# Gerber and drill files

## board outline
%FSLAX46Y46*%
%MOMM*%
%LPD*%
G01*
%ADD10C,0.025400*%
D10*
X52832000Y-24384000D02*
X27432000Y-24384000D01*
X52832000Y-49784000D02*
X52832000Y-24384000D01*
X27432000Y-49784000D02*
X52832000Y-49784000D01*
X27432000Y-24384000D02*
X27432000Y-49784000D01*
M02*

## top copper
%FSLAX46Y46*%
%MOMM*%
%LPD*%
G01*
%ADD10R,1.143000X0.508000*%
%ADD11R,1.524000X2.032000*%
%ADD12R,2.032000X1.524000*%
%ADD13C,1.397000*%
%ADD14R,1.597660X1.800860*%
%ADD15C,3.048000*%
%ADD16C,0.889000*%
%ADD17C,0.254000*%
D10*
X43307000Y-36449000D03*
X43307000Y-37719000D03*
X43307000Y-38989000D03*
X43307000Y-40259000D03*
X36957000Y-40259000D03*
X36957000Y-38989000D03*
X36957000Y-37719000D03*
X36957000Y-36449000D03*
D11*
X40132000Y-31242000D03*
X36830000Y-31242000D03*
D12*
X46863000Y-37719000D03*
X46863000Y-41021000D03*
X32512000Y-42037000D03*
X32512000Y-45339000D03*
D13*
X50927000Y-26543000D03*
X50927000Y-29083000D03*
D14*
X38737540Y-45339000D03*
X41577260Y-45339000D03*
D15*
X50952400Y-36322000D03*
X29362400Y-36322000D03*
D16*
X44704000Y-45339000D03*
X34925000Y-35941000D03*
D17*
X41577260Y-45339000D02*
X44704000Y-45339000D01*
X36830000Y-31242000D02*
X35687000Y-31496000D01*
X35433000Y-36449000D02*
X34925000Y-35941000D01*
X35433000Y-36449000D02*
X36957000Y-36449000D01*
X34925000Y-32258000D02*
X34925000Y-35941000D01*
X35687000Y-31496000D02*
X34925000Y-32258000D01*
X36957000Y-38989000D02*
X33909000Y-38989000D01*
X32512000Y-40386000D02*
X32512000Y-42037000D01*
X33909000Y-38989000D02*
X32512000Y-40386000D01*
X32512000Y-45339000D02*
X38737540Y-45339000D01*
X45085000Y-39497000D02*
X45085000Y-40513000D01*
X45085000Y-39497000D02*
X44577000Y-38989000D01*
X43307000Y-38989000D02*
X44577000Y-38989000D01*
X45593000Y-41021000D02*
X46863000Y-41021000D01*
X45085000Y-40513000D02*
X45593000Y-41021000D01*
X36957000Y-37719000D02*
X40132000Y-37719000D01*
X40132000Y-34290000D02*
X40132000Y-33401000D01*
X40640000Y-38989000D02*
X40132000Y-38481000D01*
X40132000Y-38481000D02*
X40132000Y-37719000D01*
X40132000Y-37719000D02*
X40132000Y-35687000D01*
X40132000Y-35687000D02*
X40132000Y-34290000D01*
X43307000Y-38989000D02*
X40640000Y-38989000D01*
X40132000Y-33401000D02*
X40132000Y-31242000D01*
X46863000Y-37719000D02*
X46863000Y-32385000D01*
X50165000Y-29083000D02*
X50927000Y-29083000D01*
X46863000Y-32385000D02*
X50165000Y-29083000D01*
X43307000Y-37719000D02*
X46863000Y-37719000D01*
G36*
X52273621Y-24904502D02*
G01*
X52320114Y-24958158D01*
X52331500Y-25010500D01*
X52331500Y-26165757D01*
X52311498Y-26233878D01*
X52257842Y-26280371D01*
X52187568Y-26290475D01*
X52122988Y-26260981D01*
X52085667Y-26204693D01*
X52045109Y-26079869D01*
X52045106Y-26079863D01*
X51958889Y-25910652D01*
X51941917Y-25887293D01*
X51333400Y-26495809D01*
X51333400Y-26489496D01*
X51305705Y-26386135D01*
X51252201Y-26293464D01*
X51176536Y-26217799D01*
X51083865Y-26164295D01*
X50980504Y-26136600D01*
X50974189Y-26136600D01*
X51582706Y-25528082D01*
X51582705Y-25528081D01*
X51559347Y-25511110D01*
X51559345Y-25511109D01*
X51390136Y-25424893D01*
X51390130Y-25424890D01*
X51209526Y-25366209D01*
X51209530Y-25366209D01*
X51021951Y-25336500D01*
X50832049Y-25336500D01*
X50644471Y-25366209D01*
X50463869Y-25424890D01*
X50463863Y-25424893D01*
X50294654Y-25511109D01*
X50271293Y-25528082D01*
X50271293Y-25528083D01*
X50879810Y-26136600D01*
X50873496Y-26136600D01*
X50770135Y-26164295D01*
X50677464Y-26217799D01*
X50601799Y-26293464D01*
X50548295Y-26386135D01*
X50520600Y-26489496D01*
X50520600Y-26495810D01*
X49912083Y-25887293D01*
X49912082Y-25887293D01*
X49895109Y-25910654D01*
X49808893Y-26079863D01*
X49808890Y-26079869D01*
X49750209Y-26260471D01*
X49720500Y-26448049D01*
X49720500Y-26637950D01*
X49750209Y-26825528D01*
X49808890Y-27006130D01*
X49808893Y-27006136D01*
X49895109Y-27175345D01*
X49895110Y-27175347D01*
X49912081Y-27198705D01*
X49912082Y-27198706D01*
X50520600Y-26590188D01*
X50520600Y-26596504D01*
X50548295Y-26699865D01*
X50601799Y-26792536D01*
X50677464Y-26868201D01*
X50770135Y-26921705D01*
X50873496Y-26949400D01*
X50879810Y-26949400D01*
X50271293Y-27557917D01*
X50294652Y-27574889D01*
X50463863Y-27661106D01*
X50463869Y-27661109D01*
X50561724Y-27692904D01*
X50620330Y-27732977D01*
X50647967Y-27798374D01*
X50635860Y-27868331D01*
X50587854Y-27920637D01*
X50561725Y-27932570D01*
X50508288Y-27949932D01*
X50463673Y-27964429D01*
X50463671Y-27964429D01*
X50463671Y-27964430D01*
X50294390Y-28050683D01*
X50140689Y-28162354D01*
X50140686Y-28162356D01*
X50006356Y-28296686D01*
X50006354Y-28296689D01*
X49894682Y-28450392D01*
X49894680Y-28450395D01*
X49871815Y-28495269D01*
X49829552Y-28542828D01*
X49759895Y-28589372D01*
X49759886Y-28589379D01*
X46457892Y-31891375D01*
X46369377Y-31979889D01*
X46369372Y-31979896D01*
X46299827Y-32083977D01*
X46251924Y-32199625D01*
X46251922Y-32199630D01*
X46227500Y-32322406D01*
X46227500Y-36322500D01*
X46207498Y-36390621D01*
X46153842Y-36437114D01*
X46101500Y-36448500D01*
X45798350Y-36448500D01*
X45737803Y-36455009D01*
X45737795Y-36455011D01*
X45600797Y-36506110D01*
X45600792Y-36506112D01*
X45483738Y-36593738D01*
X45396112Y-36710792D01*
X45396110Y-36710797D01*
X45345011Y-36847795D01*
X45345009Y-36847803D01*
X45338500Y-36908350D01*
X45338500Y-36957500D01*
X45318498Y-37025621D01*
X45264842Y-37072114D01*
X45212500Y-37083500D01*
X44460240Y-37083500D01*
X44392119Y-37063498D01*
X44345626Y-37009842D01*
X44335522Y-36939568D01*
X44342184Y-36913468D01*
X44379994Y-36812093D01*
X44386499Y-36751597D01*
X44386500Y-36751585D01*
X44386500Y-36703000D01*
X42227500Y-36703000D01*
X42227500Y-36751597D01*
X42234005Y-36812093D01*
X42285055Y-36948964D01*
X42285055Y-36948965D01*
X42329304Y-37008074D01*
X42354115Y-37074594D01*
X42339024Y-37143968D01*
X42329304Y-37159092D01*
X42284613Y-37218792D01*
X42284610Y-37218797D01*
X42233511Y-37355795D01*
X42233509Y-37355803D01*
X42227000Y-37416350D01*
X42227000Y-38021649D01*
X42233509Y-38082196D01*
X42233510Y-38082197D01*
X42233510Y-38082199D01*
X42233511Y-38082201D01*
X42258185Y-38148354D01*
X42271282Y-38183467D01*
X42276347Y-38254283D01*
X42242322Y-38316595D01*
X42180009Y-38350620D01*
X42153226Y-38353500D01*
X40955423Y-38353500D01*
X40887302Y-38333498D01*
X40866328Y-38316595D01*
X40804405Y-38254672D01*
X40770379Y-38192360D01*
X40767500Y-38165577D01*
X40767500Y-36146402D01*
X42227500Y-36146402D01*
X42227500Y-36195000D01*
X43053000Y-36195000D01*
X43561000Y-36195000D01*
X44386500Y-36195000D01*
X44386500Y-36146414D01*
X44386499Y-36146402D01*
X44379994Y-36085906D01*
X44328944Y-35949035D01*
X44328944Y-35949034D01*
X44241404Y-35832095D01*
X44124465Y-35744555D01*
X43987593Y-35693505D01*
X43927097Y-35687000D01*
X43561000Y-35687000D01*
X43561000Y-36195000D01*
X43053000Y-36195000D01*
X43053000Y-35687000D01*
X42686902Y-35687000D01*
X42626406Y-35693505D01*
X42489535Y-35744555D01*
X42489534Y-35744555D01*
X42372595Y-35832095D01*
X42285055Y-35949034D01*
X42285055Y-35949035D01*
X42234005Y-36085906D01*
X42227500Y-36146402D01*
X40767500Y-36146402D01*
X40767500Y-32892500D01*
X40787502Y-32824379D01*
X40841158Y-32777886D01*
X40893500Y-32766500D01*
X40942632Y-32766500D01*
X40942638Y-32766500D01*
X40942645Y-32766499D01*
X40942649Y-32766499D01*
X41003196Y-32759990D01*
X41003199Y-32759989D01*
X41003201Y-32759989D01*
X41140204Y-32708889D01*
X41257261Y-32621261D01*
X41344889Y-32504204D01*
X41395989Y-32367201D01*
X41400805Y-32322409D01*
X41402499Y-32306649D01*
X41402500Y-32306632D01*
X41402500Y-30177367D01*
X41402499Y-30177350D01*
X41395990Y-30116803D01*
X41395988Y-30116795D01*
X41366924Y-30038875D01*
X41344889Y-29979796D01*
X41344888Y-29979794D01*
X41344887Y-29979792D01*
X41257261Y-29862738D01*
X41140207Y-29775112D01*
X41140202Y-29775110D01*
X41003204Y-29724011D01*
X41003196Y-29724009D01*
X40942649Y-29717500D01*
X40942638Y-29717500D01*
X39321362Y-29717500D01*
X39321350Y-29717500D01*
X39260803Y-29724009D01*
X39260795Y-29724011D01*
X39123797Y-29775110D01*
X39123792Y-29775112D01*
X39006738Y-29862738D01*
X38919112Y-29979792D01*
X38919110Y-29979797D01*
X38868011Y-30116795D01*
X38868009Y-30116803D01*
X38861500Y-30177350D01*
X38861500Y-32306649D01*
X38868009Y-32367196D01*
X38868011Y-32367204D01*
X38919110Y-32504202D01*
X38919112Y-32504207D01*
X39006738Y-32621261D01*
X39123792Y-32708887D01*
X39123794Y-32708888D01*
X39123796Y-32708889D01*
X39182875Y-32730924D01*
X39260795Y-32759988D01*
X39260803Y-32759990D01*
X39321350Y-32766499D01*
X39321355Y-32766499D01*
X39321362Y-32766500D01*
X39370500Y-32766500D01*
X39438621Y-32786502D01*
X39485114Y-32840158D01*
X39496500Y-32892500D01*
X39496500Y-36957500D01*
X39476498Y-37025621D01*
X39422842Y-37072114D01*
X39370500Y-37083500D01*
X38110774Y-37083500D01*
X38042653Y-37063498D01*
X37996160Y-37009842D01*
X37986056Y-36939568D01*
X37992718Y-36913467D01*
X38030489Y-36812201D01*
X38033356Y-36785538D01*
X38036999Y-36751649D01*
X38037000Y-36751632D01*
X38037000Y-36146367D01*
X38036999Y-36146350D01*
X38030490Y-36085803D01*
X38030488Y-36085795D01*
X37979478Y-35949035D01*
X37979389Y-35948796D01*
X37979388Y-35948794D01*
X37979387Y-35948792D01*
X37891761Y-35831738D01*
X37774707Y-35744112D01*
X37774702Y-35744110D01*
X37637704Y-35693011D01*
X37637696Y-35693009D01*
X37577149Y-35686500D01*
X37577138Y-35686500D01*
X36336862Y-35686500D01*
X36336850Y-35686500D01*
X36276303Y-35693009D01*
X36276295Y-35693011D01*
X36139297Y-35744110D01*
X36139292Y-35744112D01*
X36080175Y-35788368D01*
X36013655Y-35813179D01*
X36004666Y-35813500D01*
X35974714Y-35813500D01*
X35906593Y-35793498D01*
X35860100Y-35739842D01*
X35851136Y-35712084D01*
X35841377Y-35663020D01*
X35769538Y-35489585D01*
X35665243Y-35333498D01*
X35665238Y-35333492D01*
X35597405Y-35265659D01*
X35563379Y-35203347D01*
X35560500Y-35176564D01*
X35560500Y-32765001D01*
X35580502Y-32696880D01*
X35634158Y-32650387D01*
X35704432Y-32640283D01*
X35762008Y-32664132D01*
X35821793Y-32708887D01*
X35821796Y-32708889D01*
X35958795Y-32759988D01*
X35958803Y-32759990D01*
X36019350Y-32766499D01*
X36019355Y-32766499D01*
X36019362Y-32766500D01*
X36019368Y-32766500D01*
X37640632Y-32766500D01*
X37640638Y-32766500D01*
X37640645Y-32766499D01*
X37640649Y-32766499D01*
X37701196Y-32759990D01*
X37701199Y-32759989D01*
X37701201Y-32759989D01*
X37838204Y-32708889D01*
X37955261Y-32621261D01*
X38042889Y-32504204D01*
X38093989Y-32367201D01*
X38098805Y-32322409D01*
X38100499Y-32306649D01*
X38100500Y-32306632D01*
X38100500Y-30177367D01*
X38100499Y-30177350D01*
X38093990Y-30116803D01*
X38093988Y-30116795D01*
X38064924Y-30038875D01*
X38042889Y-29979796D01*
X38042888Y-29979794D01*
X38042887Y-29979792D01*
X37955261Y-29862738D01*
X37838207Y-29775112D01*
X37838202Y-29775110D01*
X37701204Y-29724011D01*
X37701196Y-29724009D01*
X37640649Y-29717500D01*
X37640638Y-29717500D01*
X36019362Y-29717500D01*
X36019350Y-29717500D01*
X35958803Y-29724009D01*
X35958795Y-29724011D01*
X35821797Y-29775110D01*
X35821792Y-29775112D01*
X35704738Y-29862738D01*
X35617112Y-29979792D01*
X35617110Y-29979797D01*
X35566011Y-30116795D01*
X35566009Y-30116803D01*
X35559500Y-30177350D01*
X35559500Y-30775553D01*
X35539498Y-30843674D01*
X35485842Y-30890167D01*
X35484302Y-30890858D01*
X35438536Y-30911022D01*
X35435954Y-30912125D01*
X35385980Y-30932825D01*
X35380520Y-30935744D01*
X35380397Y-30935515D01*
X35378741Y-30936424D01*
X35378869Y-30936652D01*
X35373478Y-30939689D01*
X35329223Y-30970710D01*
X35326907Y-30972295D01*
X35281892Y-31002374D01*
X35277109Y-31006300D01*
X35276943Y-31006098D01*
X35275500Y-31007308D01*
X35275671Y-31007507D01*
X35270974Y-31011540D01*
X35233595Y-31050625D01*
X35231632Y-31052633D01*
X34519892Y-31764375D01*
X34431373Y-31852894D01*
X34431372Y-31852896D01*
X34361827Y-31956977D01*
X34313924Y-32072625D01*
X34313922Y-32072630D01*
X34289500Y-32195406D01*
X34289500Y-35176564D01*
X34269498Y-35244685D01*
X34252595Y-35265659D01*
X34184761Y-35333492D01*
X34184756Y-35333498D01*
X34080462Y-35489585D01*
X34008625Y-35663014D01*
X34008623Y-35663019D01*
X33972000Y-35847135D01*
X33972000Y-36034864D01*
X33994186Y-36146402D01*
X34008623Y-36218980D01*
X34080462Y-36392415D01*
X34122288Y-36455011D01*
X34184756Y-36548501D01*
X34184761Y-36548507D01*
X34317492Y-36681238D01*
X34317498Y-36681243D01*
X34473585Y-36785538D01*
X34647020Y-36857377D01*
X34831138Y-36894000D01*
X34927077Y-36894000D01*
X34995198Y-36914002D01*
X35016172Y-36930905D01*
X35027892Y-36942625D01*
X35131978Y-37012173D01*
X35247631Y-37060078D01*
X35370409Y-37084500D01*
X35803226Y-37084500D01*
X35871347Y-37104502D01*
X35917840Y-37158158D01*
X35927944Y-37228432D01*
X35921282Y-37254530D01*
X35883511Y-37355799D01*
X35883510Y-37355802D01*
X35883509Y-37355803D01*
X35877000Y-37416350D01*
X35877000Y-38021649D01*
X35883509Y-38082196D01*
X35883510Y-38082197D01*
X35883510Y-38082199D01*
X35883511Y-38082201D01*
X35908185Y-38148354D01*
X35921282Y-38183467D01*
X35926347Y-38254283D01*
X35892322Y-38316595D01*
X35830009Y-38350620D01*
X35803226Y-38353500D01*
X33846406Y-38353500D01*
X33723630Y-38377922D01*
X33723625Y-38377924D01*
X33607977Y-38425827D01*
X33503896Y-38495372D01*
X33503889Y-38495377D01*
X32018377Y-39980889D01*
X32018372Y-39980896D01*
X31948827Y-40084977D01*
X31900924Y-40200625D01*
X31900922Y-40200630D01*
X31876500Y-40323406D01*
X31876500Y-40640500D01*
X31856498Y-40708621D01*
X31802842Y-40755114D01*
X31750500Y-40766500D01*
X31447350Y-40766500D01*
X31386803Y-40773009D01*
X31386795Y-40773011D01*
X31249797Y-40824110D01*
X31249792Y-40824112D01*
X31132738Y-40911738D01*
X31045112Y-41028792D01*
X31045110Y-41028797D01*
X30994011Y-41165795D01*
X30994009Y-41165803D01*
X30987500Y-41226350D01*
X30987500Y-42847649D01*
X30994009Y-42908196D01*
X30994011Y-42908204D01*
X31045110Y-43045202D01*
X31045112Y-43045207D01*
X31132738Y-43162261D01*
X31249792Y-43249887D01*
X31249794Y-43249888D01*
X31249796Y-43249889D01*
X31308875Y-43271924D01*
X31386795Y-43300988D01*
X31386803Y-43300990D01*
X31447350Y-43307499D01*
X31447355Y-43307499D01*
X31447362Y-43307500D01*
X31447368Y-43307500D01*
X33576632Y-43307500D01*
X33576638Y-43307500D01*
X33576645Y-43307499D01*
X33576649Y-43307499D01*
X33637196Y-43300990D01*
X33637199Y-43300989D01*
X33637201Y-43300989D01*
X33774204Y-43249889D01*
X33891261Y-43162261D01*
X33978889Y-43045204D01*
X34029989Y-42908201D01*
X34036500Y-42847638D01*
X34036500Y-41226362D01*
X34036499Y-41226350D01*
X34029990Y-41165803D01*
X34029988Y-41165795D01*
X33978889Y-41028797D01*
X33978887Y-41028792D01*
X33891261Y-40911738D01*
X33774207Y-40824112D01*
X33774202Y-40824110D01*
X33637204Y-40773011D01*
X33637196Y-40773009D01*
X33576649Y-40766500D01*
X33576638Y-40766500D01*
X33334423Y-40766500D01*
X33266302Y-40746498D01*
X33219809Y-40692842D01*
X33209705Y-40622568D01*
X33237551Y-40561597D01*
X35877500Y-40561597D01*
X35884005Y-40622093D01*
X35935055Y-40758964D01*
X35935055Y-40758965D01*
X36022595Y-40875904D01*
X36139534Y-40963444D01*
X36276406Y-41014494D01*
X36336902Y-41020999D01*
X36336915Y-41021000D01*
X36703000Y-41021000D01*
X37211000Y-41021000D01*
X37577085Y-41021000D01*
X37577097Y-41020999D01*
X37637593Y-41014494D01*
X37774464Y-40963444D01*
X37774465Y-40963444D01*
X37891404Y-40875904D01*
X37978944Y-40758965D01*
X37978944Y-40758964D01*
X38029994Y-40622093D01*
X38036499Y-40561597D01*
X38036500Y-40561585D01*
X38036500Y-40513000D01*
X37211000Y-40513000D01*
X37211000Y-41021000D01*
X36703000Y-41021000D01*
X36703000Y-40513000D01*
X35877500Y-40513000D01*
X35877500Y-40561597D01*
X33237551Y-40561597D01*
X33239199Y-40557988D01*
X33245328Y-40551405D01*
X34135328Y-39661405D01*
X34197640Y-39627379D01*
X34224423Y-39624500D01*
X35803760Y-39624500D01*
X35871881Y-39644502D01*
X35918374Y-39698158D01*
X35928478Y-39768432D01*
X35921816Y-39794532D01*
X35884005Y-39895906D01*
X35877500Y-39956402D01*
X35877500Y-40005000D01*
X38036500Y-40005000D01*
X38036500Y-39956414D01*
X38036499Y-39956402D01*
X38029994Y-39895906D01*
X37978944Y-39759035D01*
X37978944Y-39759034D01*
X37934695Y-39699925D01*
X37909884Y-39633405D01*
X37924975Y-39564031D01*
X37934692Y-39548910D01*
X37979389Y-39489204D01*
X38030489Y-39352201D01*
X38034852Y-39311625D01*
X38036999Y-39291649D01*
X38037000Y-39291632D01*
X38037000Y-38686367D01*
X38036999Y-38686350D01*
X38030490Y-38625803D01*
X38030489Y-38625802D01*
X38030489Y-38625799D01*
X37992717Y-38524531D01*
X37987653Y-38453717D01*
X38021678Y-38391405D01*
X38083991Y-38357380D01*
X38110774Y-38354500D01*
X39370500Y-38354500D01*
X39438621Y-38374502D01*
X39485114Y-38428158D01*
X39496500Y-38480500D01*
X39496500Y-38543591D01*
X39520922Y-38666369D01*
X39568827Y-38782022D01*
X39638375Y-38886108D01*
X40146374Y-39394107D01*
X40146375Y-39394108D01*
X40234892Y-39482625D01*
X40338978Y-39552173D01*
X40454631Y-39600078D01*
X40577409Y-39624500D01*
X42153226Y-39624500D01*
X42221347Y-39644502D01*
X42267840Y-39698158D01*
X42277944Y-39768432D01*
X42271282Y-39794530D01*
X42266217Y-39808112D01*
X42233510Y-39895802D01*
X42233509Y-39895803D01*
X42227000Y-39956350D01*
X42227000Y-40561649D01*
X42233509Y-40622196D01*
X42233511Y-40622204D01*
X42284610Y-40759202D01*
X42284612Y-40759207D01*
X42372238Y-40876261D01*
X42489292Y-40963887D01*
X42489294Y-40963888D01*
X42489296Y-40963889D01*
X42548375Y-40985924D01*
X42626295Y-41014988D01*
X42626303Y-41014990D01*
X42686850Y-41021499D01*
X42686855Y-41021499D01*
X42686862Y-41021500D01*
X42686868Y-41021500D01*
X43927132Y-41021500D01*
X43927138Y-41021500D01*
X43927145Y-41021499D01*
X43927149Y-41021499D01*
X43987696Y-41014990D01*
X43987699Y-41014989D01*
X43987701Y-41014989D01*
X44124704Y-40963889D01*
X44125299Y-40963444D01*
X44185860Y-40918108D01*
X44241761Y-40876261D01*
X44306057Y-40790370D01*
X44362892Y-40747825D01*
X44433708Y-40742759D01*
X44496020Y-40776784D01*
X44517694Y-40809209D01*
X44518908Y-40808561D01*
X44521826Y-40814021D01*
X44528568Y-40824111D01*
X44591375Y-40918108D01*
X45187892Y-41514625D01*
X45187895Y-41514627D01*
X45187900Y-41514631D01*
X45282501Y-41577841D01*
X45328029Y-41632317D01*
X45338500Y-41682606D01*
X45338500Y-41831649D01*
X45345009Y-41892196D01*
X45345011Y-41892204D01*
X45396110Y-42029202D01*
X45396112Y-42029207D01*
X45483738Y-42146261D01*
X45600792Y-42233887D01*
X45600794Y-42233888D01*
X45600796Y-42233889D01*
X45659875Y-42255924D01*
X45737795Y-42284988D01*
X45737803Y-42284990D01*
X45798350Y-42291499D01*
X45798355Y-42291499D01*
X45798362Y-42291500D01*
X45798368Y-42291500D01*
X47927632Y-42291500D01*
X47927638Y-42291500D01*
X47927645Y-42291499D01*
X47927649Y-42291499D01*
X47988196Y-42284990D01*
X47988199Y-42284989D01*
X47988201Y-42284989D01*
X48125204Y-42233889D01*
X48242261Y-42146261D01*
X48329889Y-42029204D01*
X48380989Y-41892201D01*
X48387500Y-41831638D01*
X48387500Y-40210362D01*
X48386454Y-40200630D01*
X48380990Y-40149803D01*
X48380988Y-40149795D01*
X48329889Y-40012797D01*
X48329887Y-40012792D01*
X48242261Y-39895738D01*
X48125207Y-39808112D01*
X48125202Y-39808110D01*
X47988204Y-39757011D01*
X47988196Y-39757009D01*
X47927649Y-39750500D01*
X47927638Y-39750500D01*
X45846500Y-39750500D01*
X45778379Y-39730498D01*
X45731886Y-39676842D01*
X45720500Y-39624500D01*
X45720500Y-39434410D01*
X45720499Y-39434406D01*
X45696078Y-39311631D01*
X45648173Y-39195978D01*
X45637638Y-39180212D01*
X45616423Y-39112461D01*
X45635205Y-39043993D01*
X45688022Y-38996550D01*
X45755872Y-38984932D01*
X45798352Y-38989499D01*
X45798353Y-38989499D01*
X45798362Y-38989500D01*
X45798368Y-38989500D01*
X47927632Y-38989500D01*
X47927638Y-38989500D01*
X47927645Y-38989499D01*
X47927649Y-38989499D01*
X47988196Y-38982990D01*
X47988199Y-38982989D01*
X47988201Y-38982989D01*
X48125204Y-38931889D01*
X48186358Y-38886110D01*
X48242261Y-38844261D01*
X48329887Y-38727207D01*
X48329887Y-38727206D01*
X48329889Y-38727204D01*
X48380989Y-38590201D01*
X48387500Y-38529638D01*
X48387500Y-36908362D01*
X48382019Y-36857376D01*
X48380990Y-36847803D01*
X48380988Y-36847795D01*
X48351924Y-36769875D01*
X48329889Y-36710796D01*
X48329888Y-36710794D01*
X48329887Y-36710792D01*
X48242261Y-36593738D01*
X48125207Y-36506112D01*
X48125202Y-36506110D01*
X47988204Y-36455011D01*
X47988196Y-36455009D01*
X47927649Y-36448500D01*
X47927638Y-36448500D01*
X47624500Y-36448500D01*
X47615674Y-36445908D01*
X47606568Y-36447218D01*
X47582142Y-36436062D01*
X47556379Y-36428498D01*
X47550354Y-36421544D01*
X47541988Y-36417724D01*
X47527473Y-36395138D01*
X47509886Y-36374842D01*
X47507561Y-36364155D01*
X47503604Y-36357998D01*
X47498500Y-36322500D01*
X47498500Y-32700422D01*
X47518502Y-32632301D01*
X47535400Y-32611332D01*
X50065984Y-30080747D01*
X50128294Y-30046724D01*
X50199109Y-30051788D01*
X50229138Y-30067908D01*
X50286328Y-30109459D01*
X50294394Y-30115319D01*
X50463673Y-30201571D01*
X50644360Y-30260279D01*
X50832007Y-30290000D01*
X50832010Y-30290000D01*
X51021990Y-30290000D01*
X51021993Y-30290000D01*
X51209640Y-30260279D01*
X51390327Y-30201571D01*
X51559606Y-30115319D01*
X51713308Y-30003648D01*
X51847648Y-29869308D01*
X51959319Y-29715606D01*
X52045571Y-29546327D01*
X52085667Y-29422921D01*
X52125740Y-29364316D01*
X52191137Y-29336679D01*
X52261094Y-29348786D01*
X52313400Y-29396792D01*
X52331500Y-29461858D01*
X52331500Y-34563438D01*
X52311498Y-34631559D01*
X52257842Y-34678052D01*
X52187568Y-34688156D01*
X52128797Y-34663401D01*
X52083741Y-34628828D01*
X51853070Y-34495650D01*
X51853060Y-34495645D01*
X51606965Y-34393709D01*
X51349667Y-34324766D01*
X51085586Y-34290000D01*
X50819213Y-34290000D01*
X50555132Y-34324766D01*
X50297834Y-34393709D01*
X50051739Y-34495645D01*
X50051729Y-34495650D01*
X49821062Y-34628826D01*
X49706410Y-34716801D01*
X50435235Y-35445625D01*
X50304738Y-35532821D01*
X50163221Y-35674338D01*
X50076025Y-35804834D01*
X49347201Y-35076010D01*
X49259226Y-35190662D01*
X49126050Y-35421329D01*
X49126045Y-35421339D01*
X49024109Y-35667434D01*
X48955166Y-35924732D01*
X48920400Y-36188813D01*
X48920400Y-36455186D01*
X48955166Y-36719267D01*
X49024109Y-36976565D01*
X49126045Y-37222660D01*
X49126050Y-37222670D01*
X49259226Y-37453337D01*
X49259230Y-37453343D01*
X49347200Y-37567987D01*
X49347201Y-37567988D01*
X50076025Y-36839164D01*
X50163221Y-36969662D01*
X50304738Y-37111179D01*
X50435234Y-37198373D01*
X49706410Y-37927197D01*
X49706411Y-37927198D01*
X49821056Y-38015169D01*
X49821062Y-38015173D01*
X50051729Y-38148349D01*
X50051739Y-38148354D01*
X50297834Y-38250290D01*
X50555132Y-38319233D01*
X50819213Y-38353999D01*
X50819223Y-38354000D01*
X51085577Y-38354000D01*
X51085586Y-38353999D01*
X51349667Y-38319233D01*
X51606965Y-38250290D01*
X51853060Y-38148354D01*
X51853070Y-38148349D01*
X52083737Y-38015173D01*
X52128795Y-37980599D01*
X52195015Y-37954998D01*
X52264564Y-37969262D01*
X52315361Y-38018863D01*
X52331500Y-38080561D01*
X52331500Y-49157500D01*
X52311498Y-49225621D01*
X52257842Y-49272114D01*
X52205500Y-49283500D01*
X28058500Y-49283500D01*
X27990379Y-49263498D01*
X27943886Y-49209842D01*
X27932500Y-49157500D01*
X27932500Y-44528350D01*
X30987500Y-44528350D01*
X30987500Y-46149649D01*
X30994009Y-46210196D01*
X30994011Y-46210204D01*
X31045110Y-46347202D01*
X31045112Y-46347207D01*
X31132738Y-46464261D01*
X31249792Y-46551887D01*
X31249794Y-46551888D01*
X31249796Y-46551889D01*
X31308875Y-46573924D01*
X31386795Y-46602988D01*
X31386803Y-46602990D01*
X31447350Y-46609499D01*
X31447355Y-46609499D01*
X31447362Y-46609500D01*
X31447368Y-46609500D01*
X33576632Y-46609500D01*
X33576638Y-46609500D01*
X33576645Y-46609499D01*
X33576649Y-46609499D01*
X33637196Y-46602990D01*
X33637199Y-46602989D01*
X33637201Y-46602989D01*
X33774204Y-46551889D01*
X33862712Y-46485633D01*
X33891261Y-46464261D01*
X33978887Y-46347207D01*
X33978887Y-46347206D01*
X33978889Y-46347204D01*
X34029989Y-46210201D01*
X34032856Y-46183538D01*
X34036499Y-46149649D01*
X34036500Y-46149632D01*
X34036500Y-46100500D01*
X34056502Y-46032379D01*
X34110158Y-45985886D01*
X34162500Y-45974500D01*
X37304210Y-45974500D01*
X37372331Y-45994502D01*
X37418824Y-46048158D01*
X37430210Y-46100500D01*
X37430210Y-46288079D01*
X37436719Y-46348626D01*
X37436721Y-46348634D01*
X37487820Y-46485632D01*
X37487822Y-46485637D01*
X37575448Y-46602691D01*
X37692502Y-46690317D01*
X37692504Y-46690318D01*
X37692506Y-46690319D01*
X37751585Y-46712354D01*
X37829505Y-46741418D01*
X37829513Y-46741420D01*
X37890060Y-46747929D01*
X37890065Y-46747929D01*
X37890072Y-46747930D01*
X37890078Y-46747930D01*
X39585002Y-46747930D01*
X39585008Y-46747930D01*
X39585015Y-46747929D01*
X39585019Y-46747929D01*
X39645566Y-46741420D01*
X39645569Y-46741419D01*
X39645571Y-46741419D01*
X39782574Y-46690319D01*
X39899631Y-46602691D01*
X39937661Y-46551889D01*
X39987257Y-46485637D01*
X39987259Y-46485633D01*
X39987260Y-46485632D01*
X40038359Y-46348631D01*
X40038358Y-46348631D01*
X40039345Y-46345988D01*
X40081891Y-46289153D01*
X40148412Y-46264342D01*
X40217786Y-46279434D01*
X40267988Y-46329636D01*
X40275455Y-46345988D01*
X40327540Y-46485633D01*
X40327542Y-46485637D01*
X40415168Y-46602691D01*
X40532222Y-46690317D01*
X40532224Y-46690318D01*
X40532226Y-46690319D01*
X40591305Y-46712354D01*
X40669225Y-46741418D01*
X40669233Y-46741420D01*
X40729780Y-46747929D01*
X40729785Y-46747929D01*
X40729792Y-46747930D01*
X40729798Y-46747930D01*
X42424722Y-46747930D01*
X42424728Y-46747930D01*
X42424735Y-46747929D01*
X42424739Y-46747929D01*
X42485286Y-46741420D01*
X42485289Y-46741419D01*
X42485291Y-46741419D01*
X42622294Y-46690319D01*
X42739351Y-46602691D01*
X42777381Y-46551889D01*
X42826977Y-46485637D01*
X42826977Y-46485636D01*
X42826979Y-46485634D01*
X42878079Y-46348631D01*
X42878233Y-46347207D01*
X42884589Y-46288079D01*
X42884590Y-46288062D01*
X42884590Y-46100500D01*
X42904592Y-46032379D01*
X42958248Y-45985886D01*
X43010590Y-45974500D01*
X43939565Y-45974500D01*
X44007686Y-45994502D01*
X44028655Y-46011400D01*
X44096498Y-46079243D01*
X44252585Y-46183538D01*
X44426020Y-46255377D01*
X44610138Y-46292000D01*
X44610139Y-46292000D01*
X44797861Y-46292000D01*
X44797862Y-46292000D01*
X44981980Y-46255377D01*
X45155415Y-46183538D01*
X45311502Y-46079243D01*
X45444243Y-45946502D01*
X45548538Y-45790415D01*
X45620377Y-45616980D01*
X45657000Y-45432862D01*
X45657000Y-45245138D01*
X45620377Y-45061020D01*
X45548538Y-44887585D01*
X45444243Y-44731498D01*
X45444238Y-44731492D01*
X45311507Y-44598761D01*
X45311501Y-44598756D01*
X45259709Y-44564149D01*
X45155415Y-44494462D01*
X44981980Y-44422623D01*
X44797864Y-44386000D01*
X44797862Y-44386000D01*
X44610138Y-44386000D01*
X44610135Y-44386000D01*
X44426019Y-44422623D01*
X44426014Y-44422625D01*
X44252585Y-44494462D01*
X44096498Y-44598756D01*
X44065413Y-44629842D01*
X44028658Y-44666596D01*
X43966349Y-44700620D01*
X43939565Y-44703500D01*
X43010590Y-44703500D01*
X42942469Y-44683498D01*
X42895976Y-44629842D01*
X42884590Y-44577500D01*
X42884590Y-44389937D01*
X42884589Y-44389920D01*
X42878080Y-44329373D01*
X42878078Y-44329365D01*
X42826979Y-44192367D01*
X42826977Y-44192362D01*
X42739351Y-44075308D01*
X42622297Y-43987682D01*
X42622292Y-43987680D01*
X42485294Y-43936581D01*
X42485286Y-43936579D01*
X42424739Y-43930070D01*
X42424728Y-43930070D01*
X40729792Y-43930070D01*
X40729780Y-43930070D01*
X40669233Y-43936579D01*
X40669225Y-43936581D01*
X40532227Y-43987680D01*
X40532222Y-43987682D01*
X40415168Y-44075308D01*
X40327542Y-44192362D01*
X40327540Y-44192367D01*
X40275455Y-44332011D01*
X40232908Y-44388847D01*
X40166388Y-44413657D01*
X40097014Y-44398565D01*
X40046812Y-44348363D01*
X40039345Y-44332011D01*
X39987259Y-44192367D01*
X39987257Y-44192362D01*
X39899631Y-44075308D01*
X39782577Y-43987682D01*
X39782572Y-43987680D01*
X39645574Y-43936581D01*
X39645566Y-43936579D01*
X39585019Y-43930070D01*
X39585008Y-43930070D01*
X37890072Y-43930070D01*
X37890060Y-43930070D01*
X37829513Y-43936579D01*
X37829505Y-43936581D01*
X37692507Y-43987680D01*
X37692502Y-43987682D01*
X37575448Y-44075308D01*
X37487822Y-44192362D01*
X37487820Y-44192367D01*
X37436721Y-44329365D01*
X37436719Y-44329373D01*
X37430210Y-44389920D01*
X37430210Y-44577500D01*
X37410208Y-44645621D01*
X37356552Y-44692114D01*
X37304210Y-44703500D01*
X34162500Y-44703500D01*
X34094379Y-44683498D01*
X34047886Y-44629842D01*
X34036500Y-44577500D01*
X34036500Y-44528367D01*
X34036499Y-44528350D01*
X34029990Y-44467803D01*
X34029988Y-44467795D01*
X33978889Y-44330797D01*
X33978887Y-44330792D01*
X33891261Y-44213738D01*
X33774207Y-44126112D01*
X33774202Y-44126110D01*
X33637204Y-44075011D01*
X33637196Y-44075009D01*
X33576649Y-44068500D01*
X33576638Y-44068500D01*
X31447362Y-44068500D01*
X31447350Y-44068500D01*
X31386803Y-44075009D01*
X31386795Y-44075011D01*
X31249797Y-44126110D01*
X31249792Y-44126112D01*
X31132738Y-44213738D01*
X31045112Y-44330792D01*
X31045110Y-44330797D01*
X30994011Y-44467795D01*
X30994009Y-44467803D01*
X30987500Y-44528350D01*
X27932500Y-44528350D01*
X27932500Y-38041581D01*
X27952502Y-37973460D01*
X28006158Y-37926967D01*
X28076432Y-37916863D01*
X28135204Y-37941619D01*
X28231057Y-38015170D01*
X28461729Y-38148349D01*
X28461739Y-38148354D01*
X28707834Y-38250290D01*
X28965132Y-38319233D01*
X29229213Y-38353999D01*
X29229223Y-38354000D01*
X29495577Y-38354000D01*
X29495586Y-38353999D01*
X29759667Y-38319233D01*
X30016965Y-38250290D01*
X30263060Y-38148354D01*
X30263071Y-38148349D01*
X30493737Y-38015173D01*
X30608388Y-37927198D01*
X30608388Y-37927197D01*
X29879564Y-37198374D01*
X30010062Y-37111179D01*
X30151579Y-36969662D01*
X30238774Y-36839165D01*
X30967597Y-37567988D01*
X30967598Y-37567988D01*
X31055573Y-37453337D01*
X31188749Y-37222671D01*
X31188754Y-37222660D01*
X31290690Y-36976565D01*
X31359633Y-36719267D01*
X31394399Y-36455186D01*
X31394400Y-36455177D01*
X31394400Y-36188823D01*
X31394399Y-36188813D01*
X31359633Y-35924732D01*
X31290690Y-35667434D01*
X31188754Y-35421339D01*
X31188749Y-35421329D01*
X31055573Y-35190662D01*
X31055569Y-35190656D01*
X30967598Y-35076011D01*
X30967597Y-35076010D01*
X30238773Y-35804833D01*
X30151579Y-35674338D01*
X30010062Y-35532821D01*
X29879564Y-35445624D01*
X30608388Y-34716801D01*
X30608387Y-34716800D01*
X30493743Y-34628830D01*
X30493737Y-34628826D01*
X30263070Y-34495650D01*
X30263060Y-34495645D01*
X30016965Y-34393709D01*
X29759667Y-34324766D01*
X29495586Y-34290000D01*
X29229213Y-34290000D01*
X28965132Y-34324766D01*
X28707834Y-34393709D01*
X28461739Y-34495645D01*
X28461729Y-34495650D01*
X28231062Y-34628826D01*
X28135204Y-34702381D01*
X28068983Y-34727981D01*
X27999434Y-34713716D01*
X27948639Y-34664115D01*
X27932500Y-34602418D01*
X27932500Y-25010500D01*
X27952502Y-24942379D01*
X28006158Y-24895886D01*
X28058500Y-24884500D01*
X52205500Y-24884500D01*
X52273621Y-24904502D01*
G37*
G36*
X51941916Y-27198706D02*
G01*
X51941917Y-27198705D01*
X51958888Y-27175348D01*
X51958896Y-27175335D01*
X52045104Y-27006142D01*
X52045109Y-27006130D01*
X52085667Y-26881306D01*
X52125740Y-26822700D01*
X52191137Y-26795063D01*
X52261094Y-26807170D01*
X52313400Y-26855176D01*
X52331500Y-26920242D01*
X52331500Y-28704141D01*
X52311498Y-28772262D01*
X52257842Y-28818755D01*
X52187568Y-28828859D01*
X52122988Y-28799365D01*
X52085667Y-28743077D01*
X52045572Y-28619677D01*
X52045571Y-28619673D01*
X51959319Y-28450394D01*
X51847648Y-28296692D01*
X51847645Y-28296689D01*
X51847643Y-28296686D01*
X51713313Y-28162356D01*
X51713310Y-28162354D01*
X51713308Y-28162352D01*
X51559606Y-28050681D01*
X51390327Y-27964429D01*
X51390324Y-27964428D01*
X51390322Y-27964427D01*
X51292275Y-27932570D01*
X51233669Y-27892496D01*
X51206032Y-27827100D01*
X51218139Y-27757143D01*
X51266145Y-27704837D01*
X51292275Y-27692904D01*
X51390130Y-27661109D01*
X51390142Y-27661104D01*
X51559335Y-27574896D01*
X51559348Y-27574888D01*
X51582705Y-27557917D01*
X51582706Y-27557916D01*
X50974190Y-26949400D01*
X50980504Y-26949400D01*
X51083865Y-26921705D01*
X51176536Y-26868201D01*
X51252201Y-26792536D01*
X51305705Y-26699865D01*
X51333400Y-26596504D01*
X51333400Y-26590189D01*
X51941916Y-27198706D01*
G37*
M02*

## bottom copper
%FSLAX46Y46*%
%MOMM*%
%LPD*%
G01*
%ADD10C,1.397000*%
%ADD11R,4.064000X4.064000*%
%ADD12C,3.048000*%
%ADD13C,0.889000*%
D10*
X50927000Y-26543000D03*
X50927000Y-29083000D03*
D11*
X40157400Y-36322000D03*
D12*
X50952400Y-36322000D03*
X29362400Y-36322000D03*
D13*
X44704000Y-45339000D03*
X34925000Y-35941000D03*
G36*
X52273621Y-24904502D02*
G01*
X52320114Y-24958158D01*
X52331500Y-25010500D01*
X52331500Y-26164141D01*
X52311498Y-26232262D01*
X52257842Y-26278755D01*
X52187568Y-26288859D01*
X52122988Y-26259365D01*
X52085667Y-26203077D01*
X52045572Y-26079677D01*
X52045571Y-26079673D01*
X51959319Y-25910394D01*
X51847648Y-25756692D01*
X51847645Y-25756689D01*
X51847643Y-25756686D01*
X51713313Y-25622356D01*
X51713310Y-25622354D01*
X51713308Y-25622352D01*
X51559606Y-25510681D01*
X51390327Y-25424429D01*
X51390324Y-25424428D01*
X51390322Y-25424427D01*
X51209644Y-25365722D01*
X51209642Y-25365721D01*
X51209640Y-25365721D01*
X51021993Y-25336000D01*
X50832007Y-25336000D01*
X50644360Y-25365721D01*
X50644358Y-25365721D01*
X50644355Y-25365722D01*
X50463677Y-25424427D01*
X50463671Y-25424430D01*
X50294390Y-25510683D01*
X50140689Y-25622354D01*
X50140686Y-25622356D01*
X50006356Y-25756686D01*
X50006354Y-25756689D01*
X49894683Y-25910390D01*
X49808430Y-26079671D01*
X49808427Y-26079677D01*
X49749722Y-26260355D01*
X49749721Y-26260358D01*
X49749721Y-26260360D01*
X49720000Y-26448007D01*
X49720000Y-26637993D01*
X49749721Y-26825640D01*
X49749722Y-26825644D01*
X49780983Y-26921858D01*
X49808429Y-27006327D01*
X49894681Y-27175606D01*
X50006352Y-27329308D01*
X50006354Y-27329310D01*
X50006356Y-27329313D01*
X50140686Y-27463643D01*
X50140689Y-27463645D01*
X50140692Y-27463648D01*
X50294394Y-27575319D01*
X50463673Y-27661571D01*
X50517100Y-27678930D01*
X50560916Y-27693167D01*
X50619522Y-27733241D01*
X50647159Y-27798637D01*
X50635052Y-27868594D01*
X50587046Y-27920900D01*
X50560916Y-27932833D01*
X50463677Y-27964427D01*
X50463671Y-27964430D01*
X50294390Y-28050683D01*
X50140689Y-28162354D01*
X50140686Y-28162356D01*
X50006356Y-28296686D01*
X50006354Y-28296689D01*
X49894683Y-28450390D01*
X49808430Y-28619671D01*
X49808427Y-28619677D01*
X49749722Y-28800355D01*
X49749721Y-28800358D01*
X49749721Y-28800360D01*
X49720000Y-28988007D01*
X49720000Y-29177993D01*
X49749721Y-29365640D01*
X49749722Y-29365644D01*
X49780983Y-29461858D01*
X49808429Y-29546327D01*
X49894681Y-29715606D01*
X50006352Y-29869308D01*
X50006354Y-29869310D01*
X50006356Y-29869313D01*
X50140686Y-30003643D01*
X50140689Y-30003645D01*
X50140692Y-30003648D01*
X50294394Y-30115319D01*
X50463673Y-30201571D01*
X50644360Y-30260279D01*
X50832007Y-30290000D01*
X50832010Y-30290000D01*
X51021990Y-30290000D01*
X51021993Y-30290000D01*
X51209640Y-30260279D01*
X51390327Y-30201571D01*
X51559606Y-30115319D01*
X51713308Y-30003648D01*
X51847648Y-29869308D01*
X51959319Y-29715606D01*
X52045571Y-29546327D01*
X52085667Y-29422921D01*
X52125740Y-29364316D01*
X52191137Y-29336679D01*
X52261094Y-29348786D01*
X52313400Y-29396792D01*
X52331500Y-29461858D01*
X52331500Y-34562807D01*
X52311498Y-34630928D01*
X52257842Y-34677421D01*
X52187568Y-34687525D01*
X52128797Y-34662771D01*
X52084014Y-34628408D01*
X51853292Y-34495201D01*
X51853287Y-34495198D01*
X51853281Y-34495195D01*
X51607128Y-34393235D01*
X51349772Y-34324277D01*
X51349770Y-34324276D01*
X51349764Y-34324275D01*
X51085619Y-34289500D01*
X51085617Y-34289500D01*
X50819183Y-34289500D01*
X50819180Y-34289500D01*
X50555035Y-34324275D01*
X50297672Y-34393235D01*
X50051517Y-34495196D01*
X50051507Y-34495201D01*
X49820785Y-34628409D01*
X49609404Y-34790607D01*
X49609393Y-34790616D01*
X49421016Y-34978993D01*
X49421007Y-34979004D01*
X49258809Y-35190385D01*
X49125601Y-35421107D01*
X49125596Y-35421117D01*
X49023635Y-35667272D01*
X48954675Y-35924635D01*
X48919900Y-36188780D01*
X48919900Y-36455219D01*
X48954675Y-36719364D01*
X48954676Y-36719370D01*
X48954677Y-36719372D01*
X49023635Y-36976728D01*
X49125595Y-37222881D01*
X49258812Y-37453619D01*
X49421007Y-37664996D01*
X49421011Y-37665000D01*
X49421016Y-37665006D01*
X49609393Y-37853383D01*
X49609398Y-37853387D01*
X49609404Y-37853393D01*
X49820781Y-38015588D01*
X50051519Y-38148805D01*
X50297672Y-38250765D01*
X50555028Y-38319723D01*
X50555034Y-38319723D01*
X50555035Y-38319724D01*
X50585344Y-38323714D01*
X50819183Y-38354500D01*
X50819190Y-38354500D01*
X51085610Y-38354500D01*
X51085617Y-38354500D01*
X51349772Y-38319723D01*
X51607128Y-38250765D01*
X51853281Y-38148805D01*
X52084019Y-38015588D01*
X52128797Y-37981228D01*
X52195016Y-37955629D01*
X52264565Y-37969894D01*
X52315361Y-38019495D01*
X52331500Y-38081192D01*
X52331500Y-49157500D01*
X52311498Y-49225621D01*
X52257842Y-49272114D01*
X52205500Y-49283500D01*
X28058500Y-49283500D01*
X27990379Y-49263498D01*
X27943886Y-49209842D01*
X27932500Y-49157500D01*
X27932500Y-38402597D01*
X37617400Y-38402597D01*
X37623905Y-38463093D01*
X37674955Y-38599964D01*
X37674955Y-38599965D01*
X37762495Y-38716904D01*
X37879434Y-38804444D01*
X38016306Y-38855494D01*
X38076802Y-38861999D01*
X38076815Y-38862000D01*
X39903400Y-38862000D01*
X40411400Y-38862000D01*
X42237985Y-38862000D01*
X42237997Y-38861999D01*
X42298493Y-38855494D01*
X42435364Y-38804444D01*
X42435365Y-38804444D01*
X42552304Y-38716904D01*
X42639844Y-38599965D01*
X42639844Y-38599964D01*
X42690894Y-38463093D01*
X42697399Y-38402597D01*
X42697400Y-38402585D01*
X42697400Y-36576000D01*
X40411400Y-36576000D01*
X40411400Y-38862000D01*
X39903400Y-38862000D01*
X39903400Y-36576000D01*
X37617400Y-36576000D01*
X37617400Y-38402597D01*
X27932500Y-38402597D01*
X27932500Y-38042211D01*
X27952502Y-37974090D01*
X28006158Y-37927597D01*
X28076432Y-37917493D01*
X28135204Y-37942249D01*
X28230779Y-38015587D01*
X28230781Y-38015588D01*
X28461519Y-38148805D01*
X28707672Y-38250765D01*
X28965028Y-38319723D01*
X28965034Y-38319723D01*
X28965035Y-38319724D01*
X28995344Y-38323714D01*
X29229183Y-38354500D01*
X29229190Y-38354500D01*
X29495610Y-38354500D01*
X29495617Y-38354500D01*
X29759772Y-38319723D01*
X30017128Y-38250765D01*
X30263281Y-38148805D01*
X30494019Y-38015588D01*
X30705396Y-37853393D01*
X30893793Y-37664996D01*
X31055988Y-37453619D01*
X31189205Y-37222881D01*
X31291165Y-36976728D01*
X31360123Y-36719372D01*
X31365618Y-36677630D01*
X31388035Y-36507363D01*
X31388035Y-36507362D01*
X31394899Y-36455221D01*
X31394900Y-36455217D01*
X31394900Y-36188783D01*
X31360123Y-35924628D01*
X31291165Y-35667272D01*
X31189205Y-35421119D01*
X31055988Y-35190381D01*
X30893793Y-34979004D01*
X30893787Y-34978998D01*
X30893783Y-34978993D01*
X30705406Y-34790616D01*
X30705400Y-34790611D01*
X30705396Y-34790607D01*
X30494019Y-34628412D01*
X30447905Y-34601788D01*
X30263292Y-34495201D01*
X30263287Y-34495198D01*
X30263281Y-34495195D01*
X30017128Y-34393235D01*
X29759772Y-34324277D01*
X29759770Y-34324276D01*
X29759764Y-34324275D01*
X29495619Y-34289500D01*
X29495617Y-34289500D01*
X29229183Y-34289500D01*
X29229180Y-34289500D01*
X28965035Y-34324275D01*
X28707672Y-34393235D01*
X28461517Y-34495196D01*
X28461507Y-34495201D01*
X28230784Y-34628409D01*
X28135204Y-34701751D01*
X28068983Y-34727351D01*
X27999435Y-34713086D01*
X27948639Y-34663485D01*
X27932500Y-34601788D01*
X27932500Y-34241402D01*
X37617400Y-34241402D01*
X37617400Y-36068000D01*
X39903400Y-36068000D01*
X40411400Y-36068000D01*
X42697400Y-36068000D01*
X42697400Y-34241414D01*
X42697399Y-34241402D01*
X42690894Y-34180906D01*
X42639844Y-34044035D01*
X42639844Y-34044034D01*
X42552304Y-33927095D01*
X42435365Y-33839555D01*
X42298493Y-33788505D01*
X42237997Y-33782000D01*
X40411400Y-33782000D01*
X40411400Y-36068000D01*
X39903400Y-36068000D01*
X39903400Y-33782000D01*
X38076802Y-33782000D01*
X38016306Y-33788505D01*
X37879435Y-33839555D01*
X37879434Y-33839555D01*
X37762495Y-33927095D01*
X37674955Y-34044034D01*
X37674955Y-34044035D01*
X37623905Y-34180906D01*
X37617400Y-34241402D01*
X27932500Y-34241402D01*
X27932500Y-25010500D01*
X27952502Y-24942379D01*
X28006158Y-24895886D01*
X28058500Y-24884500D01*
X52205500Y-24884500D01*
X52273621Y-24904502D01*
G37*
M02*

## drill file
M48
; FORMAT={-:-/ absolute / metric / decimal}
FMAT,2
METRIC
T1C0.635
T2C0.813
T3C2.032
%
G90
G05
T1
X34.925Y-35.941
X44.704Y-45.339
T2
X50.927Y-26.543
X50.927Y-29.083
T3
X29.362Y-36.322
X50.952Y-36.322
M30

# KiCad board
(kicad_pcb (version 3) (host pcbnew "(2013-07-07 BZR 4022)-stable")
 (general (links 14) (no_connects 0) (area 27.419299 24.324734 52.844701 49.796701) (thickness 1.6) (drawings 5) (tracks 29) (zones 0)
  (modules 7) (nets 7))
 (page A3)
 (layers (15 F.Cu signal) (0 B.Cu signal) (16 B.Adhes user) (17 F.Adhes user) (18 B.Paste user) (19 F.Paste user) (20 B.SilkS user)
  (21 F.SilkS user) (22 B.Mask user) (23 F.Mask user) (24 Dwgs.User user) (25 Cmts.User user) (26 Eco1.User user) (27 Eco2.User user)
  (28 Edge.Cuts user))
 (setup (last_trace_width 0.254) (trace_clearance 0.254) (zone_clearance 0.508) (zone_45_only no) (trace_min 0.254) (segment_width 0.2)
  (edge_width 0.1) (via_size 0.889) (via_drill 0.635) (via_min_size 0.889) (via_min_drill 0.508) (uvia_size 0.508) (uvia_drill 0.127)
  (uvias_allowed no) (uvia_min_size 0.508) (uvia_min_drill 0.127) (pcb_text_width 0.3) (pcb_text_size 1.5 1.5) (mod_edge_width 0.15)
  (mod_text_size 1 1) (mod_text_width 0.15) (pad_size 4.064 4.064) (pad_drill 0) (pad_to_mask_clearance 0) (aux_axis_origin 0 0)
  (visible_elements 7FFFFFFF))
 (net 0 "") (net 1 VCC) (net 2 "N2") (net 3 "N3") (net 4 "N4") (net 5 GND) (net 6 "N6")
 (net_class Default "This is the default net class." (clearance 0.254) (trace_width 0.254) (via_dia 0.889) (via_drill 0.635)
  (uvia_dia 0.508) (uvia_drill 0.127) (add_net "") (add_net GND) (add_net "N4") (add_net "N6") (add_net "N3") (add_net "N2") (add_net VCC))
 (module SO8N (layer F.Cu) (at 40.132 38.354 270)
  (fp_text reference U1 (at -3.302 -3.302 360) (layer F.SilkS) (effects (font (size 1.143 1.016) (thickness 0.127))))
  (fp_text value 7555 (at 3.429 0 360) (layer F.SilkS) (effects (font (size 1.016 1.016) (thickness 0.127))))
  (pad 8 smd rect (at -1.905 -3.175 270) (size 0.508 1.143) (layers F.Cu F.Paste F.Mask) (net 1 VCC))
  (pad 7 smd rect (at -0.635 -3.175 270) (size 0.508 1.143) (layers F.Cu F.Paste F.Mask) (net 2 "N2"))
  (pad 6 smd rect (at 0.635 -3.175 270) (size 0.508 1.143) (layers F.Cu F.Paste F.Mask) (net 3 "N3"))
  (pad 5 smd rect (at 1.905 -3.175 270) (size 0.508 1.143) (layers F.Cu F.Paste F.Mask))
  (pad 4 smd rect (at 1.905 3.175 270) (size 0.508 1.143) (layers F.Cu F.Paste F.Mask) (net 1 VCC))
  (pad 3 smd rect (at 0.635 3.175 270) (size 0.508 1.143) (layers F.Cu F.Paste F.Mask) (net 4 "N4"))
  (pad 2 smd rect (at -0.635 3.175 270) (size 0.508 1.143) (layers F.Cu F.Paste F.Mask) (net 3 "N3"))
  (pad 1 smd rect (at -1.905 3.175 270) (size 0.508 1.143) (layers F.Cu F.Paste F.Mask) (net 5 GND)))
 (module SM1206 (layer F.Cu) (at 38.481 31.242 180)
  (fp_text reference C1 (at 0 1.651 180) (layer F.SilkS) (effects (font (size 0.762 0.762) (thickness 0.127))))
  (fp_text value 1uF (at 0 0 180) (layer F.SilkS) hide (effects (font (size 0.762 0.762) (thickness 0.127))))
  (pad 1 smd rect (at -1.651 0 180) (size 1.524 2.032) (layers F.Cu F.Paste F.Mask) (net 3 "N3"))
  (pad 2 smd rect (at 1.651 0 180) (size 1.524 2.032) (layers F.Cu F.Paste F.Mask) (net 5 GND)))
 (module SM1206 (layer F.Cu) (at 46.863 39.37 270)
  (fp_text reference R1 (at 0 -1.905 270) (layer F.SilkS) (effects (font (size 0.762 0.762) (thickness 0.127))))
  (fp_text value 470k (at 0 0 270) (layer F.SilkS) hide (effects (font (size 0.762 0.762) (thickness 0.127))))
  (pad 1 smd rect (at -1.651 0 270) (size 1.524 2.032) (layers F.Cu F.Paste F.Mask) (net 2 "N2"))
  (pad 2 smd rect (at 1.651 0 270) (size 1.524 2.032) (layers F.Cu F.Paste F.Mask) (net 3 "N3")))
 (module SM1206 (layer F.Cu) (at 32.512 43.688 270)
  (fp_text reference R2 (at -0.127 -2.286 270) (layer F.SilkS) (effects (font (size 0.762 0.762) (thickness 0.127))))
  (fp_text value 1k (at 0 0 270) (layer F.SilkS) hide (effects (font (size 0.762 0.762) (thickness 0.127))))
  (pad 1 smd rect (at -1.651 0 270) (size 1.524 2.032) (layers F.Cu F.Paste F.Mask) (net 4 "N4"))
  (pad 2 smd rect (at 1.651 0 270) (size 1.524 2.032) (layers F.Cu F.Paste F.Mask) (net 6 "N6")))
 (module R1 (layer F.Cu) (at 50.927 27.813 270) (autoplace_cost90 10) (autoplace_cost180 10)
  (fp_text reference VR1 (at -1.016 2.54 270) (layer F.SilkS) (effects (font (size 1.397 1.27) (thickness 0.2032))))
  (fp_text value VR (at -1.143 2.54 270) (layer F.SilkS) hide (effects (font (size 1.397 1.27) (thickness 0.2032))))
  (pad 1 thru_hole circle (at -1.27 0 270) (size 1.397 1.397) (drill 0.8128) (layers *.Cu *.Mask F.SilkS) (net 1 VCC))
  (pad 2 thru_hole circle (at 1.27 0 270) (size 1.397 1.397) (drill 0.8128) (layers *.Cu *.Mask F.SilkS) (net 2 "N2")))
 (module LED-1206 (layer F.Cu) (at 40.1574 45.339)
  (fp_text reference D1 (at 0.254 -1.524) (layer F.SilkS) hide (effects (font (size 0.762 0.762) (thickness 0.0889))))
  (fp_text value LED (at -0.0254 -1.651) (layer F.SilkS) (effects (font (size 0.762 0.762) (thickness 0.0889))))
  (pad 1 smd rect (at -1.41986 0) (size 1.59766 1.80086) (layers F.Cu F.Paste F.Mask) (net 6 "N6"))
  (pad 2 smd rect (at 1.41986 0) (size 1.59766 1.80086) (layers F.Cu F.Paste F.Mask) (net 5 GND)))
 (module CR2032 (layer B.Cu) (at 40.1574 36.322 180)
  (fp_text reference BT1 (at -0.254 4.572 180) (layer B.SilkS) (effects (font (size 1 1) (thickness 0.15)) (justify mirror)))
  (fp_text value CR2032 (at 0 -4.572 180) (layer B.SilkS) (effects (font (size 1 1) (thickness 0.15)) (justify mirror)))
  (pad 2 smd rect (at 0 0 180) (size 4.064 4.064) (layers B.Cu B.Paste B.Mask) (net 5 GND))
  (pad 1 thru_hole circle (at -10.795 0 180) (size 3.048 3.048) (drill 2.032) (layers *.Cu *.Mask B.SilkS) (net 1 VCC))
  (pad 1 thru_hole circle (at 10.795 0 180) (size 3.048 3.048) (drill 2.032) (layers *.Cu *.Mask B.SilkS) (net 1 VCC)))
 (gr_line (start 52.832 24.384) (end 27.432 24.384) (angle 90) (layer Edge.Cuts) (width 0.0254))
 (gr_line (start 52.832 49.784) (end 52.832 24.384) (angle 90) (layer Edge.Cuts) (width 0.0254))
 (gr_line (start 27.432 49.784) (end 52.832 49.784) (angle 90) (layer Edge.Cuts) (width 0.0254))
 (gr_line (start 27.432 24.384) (end 27.432 49.784) (angle 90) (layer Edge.Cuts) (width 0.0254))
 (segment (start 41.57726 45.339) (end 44.704 45.339) (width 0.254) (layer F.Cu) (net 5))
 (via (at 44.704 45.339) (size 0.889) (layers F.Cu B.Cu) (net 5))
 (segment (start 36.83 31.242) (end 35.687 31.496) (width 0.254) (layer F.Cu) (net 5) (status 10))
 (segment (start 35.433 36.449) (end 34.925 35.941) (width 0.254) (layer F.Cu) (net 5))
 (via (at 34.925 35.941) (size 0.889) (layers F.Cu B.Cu) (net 5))
 (segment (start 35.433 36.449) (end 36.957 36.449) (width 0.254) (layer F.Cu) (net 5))
 (segment (start 34.925 32.258) (end 34.925 35.941) (width 0.254) (layer F.Cu) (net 5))
 (segment (start 35.687 31.496) (end 34.925 32.258) (width 0.254) (layer F.Cu) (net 5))
 (segment (start 36.957 38.989) (end 33.909 38.989) (width 0.254) (layer F.Cu) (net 4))
 (segment (start 32.512 40.386) (end 32.512 42.037) (width 0.254) (layer F.Cu) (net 4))
 (segment (start 33.909 38.989) (end 32.512 40.386) (width 0.254) (layer F.Cu) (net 4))
 (segment (start 32.512 45.339) (end 38.73754 45.339) (width 0.254) (layer F.Cu) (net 6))
 (segment (start 45.085 39.497) (end 45.085 40.513) (width 0.254) (layer F.Cu) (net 3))
 (segment (start 45.085 39.497) (end 44.577 38.989) (width 0.254) (layer F.Cu) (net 3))
 (segment (start 43.307 38.989) (end 44.577 38.989) (width 0.254) (layer F.Cu) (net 3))
 (segment (start 45.593 41.021) (end 46.863 41.021) (width 0.254) (layer F.Cu) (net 3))
 (segment (start 45.085 40.513) (end 45.593 41.021) (width 0.254) (layer F.Cu) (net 3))
 (segment (start 36.957 37.719) (end 40.132 37.719) (width 0.254) (layer F.Cu) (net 3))
 (segment (start 40.132 34.29) (end 40.132 33.401) (width 0.254) (layer F.Cu) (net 3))
 (segment (start 40.64 38.989) (end 40.132 38.481) (width 0.254) (layer F.Cu) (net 3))
 (segment (start 40.132 38.481) (end 40.132 37.719) (width 0.254) (layer F.Cu) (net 3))
 (segment (start 40.132 37.719) (end 40.132 35.687) (width 0.254) (layer F.Cu) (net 3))
 (segment (start 40.132 35.687) (end 40.132 34.29) (width 0.254) (layer F.Cu) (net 3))
 (segment (start 43.307 38.989) (end 40.64 38.989) (width 0.254) (layer F.Cu) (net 3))
 (segment (start 40.132 33.401) (end 40.132 31.242) (width 0.254) (layer F.Cu) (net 3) (status 20))
 (segment (start 46.863 37.719) (end 46.863 32.385) (width 0.254) (layer F.Cu) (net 2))
 (segment (start 50.165 29.083) (end 50.927 29.083) (width 0.254) (layer F.Cu) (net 2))
 (segment (start 46.863 32.385) (end 50.165 29.083) (width 0.254) (layer F.Cu) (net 2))
 (segment (start 43.307 37.719) (end 46.863 37.719) (width 0.254) (layer F.Cu) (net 2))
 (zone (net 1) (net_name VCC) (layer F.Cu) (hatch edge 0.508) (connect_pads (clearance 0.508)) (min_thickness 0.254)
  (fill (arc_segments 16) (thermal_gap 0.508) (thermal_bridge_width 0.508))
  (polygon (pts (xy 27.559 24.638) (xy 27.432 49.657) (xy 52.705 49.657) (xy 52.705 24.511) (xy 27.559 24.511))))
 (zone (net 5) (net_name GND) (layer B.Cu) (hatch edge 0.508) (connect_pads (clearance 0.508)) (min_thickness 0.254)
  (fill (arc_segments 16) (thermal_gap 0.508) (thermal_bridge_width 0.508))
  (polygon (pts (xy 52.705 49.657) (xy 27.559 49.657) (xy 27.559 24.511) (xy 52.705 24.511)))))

